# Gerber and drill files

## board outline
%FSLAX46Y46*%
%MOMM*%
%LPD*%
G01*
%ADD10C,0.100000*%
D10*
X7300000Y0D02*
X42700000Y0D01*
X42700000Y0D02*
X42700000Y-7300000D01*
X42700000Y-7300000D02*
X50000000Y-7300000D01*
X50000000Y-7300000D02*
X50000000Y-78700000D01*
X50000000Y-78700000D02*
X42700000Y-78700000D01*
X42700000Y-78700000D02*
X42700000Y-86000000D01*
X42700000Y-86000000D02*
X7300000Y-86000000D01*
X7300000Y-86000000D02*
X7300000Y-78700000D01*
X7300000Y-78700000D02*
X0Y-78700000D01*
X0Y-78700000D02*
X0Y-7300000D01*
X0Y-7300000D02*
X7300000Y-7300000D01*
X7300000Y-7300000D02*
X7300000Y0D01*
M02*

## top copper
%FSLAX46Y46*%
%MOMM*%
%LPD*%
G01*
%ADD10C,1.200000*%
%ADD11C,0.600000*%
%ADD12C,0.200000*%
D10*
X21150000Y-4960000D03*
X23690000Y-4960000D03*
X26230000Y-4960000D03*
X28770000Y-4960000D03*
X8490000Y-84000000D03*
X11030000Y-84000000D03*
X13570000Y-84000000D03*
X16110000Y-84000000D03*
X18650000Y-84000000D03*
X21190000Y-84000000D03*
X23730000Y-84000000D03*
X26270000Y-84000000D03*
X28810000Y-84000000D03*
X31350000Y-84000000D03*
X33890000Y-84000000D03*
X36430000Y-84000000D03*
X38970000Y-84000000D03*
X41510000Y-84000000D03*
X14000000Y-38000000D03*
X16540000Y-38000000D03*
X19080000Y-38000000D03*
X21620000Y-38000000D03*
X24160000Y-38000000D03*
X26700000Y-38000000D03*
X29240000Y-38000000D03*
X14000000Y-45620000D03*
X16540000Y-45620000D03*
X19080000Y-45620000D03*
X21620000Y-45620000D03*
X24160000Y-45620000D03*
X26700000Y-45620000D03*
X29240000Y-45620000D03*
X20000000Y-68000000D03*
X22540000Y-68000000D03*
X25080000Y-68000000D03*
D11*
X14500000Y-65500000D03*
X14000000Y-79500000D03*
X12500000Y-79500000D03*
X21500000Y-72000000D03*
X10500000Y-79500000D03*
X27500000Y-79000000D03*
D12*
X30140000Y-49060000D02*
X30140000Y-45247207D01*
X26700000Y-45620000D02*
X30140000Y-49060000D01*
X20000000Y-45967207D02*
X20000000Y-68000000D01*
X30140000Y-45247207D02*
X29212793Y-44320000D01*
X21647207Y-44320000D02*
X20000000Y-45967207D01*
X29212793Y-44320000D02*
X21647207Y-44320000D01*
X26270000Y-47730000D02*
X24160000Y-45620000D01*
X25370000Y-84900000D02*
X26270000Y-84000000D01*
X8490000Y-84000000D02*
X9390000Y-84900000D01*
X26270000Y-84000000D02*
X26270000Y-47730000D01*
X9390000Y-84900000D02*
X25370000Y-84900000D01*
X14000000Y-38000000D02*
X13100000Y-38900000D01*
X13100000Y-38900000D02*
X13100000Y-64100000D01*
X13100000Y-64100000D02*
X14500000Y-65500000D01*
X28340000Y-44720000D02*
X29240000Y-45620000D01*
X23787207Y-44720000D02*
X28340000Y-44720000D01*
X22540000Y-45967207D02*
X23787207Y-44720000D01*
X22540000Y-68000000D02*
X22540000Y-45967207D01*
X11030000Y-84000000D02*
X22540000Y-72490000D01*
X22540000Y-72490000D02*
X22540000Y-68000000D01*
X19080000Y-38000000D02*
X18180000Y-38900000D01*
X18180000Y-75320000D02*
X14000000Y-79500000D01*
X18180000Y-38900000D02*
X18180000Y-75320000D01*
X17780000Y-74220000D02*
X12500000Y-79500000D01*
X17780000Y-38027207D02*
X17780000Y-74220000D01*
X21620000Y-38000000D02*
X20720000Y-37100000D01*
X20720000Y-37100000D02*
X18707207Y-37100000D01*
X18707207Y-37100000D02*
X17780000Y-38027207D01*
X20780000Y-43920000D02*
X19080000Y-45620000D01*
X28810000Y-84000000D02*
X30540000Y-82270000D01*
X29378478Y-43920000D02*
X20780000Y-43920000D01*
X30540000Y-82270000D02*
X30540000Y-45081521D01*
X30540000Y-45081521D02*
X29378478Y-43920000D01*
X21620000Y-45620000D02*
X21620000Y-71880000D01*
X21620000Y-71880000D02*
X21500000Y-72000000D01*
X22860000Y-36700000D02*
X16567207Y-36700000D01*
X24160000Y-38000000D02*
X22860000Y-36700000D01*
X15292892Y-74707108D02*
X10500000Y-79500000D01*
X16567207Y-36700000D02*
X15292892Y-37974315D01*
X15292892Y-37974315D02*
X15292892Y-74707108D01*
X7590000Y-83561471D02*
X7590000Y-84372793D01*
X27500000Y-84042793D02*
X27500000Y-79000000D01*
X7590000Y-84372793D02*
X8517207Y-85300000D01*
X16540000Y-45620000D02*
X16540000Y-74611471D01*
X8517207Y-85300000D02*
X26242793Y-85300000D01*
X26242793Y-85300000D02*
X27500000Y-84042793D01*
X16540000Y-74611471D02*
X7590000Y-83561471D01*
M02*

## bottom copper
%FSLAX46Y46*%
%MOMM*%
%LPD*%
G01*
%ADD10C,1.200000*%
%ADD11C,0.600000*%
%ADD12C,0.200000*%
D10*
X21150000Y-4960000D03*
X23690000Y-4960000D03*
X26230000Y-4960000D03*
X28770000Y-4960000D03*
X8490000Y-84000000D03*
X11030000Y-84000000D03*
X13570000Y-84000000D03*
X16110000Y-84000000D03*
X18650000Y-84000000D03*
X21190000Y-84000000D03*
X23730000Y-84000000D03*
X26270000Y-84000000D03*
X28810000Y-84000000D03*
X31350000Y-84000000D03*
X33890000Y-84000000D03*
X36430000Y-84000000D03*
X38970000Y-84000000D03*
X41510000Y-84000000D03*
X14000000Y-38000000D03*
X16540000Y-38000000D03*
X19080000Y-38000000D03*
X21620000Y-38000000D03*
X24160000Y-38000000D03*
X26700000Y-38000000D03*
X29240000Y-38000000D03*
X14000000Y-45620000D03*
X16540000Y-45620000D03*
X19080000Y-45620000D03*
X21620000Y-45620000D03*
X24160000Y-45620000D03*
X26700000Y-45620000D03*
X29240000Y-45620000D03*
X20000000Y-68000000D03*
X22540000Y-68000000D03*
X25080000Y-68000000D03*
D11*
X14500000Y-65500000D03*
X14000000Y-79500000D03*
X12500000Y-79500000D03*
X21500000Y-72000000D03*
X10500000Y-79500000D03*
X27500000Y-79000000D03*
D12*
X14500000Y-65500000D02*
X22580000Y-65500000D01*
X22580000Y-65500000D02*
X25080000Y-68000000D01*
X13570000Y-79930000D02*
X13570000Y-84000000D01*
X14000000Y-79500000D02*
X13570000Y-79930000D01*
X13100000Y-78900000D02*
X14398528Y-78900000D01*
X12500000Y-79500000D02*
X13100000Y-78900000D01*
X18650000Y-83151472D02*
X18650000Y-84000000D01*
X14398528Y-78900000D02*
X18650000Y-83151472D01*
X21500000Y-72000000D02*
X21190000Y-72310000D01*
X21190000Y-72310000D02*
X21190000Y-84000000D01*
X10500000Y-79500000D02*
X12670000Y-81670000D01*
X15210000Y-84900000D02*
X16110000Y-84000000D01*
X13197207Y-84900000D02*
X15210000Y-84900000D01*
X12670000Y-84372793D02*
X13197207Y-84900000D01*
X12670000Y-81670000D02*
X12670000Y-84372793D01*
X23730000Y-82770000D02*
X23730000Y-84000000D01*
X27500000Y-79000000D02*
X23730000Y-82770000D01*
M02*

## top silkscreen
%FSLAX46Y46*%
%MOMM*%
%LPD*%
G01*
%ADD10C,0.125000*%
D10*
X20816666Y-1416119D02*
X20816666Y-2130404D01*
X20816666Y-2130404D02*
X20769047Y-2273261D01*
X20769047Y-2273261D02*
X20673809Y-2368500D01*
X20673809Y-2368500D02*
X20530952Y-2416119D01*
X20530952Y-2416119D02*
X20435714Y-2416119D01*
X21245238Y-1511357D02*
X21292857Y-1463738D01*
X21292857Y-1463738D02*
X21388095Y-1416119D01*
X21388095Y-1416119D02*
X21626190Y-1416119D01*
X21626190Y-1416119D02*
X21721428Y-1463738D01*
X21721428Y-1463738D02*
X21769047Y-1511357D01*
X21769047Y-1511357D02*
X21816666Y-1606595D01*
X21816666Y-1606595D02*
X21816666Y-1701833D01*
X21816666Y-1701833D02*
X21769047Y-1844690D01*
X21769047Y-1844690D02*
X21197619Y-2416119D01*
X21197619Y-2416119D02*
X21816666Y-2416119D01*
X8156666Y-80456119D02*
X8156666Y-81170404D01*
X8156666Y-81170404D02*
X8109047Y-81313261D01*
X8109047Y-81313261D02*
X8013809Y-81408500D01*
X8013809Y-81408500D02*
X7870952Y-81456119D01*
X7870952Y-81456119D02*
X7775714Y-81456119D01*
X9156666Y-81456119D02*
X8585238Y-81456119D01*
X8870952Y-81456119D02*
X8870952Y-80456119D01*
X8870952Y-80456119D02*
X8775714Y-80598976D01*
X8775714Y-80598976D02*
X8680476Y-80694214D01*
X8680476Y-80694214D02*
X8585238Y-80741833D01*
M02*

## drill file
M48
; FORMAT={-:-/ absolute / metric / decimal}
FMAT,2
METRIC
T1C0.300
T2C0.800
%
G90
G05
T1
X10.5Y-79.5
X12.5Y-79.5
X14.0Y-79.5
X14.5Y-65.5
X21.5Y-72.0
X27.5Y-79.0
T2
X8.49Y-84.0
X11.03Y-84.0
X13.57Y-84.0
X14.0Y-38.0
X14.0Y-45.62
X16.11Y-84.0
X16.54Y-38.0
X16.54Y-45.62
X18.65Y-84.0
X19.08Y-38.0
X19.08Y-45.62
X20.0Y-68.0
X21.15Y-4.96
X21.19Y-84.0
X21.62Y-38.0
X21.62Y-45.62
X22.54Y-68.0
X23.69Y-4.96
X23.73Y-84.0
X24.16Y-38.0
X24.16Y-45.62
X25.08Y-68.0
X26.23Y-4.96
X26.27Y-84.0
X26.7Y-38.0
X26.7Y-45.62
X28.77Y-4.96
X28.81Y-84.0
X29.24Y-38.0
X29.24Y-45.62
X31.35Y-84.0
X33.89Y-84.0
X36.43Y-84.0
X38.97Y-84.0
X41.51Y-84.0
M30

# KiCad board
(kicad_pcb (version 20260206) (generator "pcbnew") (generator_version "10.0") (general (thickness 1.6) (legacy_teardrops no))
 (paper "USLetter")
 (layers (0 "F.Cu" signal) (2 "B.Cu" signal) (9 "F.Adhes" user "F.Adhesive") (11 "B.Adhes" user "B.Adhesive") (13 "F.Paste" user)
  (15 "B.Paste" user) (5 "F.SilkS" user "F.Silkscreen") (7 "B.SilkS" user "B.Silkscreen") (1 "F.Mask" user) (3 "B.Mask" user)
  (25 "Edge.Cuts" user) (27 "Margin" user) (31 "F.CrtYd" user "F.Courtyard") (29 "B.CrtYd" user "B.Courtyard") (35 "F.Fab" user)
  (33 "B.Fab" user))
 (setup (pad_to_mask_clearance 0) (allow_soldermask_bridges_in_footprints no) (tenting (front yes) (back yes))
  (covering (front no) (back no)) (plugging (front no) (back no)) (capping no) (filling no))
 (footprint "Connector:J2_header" (layer "F.Cu") (at 21.15 4.96)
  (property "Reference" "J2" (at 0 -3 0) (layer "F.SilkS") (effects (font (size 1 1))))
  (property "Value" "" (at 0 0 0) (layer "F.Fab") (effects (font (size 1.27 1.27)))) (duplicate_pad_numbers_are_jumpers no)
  (pad "1" thru_hole circle (at 0 0) (size 1.2 1.2) (drill 0.8) (layers "*.Cu" "*.Mask") (remove_unused_layers no))
  (pad "2" thru_hole circle (at 2.54 0) (size 1.2 1.2) (drill 0.8) (layers "*.Cu" "*.Mask") (remove_unused_layers no))
  (pad "3" thru_hole circle (at 5.08 0) (size 1.2 1.2) (drill 0.8) (layers "*.Cu" "*.Mask") (remove_unused_layers no))
  (pad "4" thru_hole circle (at 7.62 0) (size 1.2 1.2) (drill 0.8) (layers "*.Cu" "*.Mask") (remove_unused_layers no)))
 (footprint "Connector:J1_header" (layer "F.Cu") (at 8.49 84)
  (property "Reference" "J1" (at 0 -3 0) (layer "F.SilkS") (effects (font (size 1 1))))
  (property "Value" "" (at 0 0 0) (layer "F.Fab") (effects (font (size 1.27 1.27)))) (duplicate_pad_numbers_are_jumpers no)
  (pad "1" thru_hole circle (at 0 0) (size 1.2 1.2) (drill 0.8) (layers "*.Cu" "*.Mask") (remove_unused_layers no) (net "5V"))
  (pad "2" thru_hole circle (at 2.54 0) (size 1.2 1.2) (drill 0.8) (layers "*.Cu" "*.Mask") (remove_unused_layers no) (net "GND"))
  (pad "3" thru_hole circle (at 5.08 0) (size 1.2 1.2) (drill 0.8) (layers "*.Cu" "*.Mask") (remove_unused_layers no) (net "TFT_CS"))
  (pad "4" thru_hole circle (at 7.62 0) (size 1.2 1.2) (drill 0.8) (layers "*.Cu" "*.Mask") (remove_unused_layers no) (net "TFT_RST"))
  (pad "5" thru_hole circle (at 10.16 0) (size 1.2 1.2) (drill 0.8) (layers "*.Cu" "*.Mask") (remove_unused_layers no) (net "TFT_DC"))
  (pad "6" thru_hole circle (at 12.7 0) (size 1.2 1.2) (drill 0.8) (layers "*.Cu" "*.Mask") (remove_unused_layers no) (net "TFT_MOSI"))
  (pad "7" thru_hole circle (at 15.24 0) (size 1.2 1.2) (drill 0.8) (layers "*.Cu" "*.Mask") (remove_unused_layers no) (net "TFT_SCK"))
  (pad "8" thru_hole circle (at 17.78 0) (size 1.2 1.2) (drill 0.8) (layers "*.Cu" "*.Mask") (remove_unused_layers no) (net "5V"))
  (pad "9" thru_hole circle (at 20.32 0) (size 1.2 1.2) (drill 0.8) (layers "*.Cu" "*.Mask") (remove_unused_layers no) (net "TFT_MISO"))
  (pad "10" thru_hole circle (at 22.86 0) (size 1.2 1.2) (drill 0.8) (layers "*.Cu" "*.Mask") (remove_unused_layers no))
  (pad "11" thru_hole circle (at 25.4 0) (size 1.2 1.2) (drill 0.8) (layers "*.Cu" "*.Mask") (remove_unused_layers no))
  (pad "12" thru_hole circle (at 27.94 0) (size 1.2 1.2) (drill 0.8) (layers "*.Cu" "*.Mask") (remove_unused_layers no))
  (pad "13" thru_hole circle (at 30.48 0) (size 1.2 1.2) (drill 0.8) (layers "*.Cu" "*.Mask") (remove_unused_layers no))
  (pad "14" thru_hole circle (at 33.02 0) (size 1.2 1.2) (drill 0.8) (layers "*.Cu" "*.Mask") (remove_unused_layers no)))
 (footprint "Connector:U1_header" (layer "B.Cu") (at 14 38)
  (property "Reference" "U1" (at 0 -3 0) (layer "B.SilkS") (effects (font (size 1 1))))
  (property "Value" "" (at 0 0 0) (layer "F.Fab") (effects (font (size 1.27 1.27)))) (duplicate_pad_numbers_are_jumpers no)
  (pad "1" thru_hole circle (at 0 0) (size 1.2 1.2) (drill 0.8) (layers "*.Cu" "*.Mask") (remove_unused_layers no) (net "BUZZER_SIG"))
  (pad "2" thru_hole circle (at 2.54 0) (size 1.2 1.2) (drill 0.8) (layers "*.Cu" "*.Mask") (remove_unused_layers no))
  (pad "3" thru_hole circle (at 5.08 0) (size 1.2 1.2) (drill 0.8) (layers "*.Cu" "*.Mask") (remove_unused_layers no) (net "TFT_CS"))
  (pad "4" thru_hole circle (at 7.62 0) (size 1.2 1.2) (drill 0.8) (layers "*.Cu" "*.Mask") (remove_unused_layers no) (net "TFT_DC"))
  (pad "5" thru_hole circle (at 10.16 0) (size 1.2 1.2) (drill 0.8) (layers "*.Cu" "*.Mask") (remove_unused_layers no) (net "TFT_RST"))
  (pad "6" thru_hole circle (at 12.7 0) (size 1.2 1.2) (drill 0.8) (layers "*.Cu" "*.Mask") (remove_unused_layers no))
  (pad "7" thru_hole circle (at 15.24 0) (size 1.2 1.2) (drill 0.8) (layers "*.Cu" "*.Mask") (remove_unused_layers no))
  (pad "8" thru_hole circle (at 0 7.62) (size 1.2 1.2) (drill 0.8) (layers "*.Cu" "*.Mask") (remove_unused_layers no))
  (pad "9" thru_hole circle (at 2.54 7.62) (size 1.2 1.2) (drill 0.8) (layers "*.Cu" "*.Mask") (remove_unused_layers no) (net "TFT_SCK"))
  (pad "10" thru_hole circle (at 5.08 7.62) (size 1.2 1.2) (drill 0.8) (layers "*.Cu" "*.Mask") (remove_unused_layers no) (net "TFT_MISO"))
  (pad "11" thru_hole circle (at 7.62 7.62) (size 1.2 1.2) (drill 0.8) (layers "*.Cu" "*.Mask") (remove_unused_layers no) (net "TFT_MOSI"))
  (pad "12" thru_hole circle (at 10.16 7.62) (size 1.2 1.2) (drill 0.8) (layers "*.Cu" "*.Mask") (remove_unused_layers no) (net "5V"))
  (pad "13" thru_hole circle (at 12.7 7.62) (size 1.2 1.2) (drill 0.8) (layers "*.Cu" "*.Mask") (remove_unused_layers no) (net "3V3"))
  (pad "14" thru_hole circle (at 15.24 7.62) (size 1.2 1.2) (drill 0.8) (layers "*.Cu" "*.Mask") (remove_unused_layers no) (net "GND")))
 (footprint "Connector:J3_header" (layer "B.Cu") (at 20 68)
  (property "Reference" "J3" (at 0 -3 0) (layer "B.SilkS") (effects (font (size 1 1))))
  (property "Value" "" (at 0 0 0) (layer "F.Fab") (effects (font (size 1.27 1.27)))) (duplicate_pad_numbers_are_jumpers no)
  (pad "1" thru_hole circle (at 0 0) (size 1.2 1.2) (drill 0.8) (layers "*.Cu" "*.Mask") (remove_unused_layers no) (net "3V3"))
  (pad "2" thru_hole circle (at 2.54 0) (size 1.2 1.2) (drill 0.8) (layers "*.Cu" "*.Mask") (remove_unused_layers no) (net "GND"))
  (pad "3" thru_hole circle (at 5.08 0) (size 1.2 1.2) (drill 0.8) (layers "*.Cu" "*.Mask") (remove_unused_layers no) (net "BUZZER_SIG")))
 (gr_line (start 7.3 0) (end 42.7 0) (stroke (width 0.1) (type default)) (layer "Edge.Cuts"))
 (gr_line (start 42.7 0) (end 42.7 7.3) (stroke (width 0.1) (type default)) (layer "Edge.Cuts"))
 (gr_line (start 42.7 7.3) (end 50 7.3) (stroke (width 0.1) (type default)) (layer "Edge.Cuts"))
 (gr_line (start 50 7.3) (end 50 78.7) (stroke (width 0.1) (type default)) (layer "Edge.Cuts"))
 (gr_line (start 50 78.7) (end 42.7 78.7) (stroke (width 0.1) (type default)) (layer "Edge.Cuts"))
 (gr_line (start 42.7 78.7) (end 42.7 86) (stroke (width 0.1) (type default)) (layer "Edge.Cuts"))
 (gr_line (start 42.7 86) (end 7.3 86) (stroke (width 0.1) (type default)) (layer "Edge.Cuts"))
 (gr_line (start 7.3 86) (end 7.3 78.7) (stroke (width 0.1) (type default)) (layer "Edge.Cuts"))
 (gr_line (start 7.3 78.7) (end 0 78.7) (stroke (width 0.1) (type default)) (layer "Edge.Cuts"))
 (gr_line (start 0 78.7) (end 0 7.3) (stroke (width 0.1) (type default)) (layer "Edge.Cuts"))
 (gr_line (start 0 7.3) (end 7.3 7.3) (stroke (width 0.1) (type default)) (layer "Edge.Cuts"))
 (gr_line (start 7.3 7.3) (end 7.3 0) (stroke (width 0.1) (type default)) (layer "Edge.Cuts"))
 (segment (start 30.14 49.06) (end 30.14 45.247207) (width 0.2) (layer "F.Cu") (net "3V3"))
 (segment (start 26.7 45.62) (end 30.14 49.06) (width 0.2) (layer "F.Cu") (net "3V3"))
 (segment (start 20 45.967207) (end 20 68) (width 0.2) (layer "F.Cu") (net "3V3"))
 (segment (start 30.14 45.247207) (end 29.212793 44.32) (width 0.2) (layer "F.Cu") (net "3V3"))
 (segment (start 21.647207 44.32) (end 20 45.967207) (width 0.2) (layer "F.Cu") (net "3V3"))
 (segment (start 29.212793 44.32) (end 21.647207 44.32) (width 0.2) (layer "F.Cu") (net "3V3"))
 (segment (start 26.27 47.73) (end 24.16 45.62) (width 0.2) (layer "F.Cu") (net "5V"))
 (segment (start 25.37 84.9) (end 26.27 84) (width 0.2) (layer "F.Cu") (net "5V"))
 (segment (start 8.49 84) (end 9.39 84.9) (width 0.2) (layer "F.Cu") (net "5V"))
 (segment (start 26.27 84) (end 26.27 47.73) (width 0.2) (layer "F.Cu") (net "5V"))
 (segment (start 9.39 84.9) (end 25.37 84.9) (width 0.2) (layer "F.Cu") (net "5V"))
 (segment (start 14 38) (end 13.1 38.9) (width 0.2) (layer "F.Cu") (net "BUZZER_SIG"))
 (segment (start 13.1 38.9) (end 13.1 64.1) (width 0.2) (layer "F.Cu") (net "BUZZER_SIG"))
 (segment (start 13.1 64.1) (end 14.5 65.5) (width 0.2) (layer "F.Cu") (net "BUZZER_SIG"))
 (via (at 14.5 65.5) (size 0.6) (drill 0.3) (layers "F.Cu" "B.Cu") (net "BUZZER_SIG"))
 (segment (start 14.5 65.5) (end 22.58 65.5) (width 0.2) (layer "B.Cu") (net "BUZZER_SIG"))
 (segment (start 22.58 65.5) (end 25.08 68) (width 0.2) (layer "B.Cu") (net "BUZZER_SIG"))
 (segment (start 28.34 44.72) (end 29.24 45.62) (width 0.2) (layer "F.Cu") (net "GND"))
 (segment (start 23.787207 44.72) (end 28.34 44.72) (width 0.2) (layer "F.Cu") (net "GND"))
 (segment (start 22.54 45.967207) (end 23.787207 44.72) (width 0.2) (layer "F.Cu") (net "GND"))
 (segment (start 22.54 68) (end 22.54 45.967207) (width 0.2) (layer "F.Cu") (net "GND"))
 (segment (start 11.03 84) (end 22.54 72.49) (width 0.2) (layer "F.Cu") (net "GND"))
 (segment (start 22.54 72.49) (end 22.54 68) (width 0.2) (layer "F.Cu") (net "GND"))
 (segment (start 19.08 38) (end 18.18 38.9) (width 0.2) (layer "F.Cu") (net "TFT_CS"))
 (segment (start 18.18 75.32) (end 14 79.5) (width 0.2) (layer "F.Cu") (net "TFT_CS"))
 (segment (start 18.18 38.9) (end 18.18 75.32) (width 0.2) (layer "F.Cu") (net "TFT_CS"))
 (via (at 14 79.5) (size 0.6) (drill 0.3) (layers "F.Cu" "B.Cu") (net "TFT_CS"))
 (segment (start 13.57 79.93) (end 13.57 84) (width 0.2) (layer "B.Cu") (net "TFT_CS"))
 (segment (start 14 79.5) (end 13.57 79.93) (width 0.2) (layer "B.Cu") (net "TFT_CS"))
 (segment (start 17.78 74.22) (end 12.5 79.5) (width 0.2) (layer "F.Cu") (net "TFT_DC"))
 (segment (start 17.78 38.027207) (end 17.78 74.22) (width 0.2) (layer "F.Cu") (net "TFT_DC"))
 (segment (start 21.62 38) (end 20.72 37.1) (width 0.2) (layer "F.Cu") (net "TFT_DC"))
 (segment (start 20.72 37.1) (end 18.707207 37.1) (width 0.2) (layer "F.Cu") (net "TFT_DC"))
 (segment (start 18.707207 37.1) (end 17.78 38.027207) (width 0.2) (layer "F.Cu") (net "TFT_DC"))
 (via (at 12.5 79.5) (size 0.6) (drill 0.3) (layers "F.Cu" "B.Cu") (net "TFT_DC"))
 (segment (start 13.1 78.9) (end 14.398528 78.9) (width 0.2) (layer "B.Cu") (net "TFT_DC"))
 (segment (start 12.5 79.5) (end 13.1 78.9) (width 0.2) (layer "B.Cu") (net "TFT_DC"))
 (segment (start 18.65 83.151472) (end 18.65 84) (width 0.2) (layer "B.Cu") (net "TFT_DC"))
 (segment (start 14.398528 78.9) (end 18.65 83.151472) (width 0.2) (layer "B.Cu") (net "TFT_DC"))
 (segment (start 20.78 43.92) (end 19.08 45.62) (width 0.2) (layer "F.Cu") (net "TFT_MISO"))
 (segment (start 28.81 84) (end 30.54 82.27) (width 0.2) (layer "F.Cu") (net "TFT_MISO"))
 (segment (start 29.378478 43.92) (end 20.78 43.92) (width 0.2) (layer "F.Cu") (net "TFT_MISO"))
 (segment (start 30.54 82.27) (end 30.54 45.081521) (width 0.2) (layer "F.Cu") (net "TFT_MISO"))
 (segment (start 30.54 45.081521) (end 29.378478 43.92) (width 0.2) (layer "F.Cu") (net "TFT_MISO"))
 (segment (start 21.62 45.62) (end 21.62 71.88) (width 0.2) (layer "F.Cu") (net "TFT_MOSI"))
 (segment (start 21.62 71.88) (end 21.5 72) (width 0.2) (layer "F.Cu") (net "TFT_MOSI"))
 (via (at 21.5 72) (size 0.6) (drill 0.3) (layers "F.Cu" "B.Cu") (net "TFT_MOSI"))
 (segment (start 21.5 72) (end 21.19 72.31) (width 0.2) (layer "B.Cu") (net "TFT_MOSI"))
 (segment (start 21.19 72.31) (end 21.19 84) (width 0.2) (layer "B.Cu") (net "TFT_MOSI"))
 (segment (start 22.86 36.7) (end 16.567207 36.7) (width 0.2) (layer "F.Cu") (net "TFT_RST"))
 (segment (start 24.16 38) (end 22.86 36.7) (width 0.2) (layer "F.Cu") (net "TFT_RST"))
 (segment (start 15.292892 74.707108) (end 10.5 79.5) (width 0.2) (layer "F.Cu") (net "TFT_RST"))
 (segment (start 16.567207 36.7) (end 15.292892 37.974315) (width 0.2) (layer "F.Cu") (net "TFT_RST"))
 (segment (start 15.292892 37.974315) (end 15.292892 74.707108) (width 0.2) (layer "F.Cu") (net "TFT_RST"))
 (via (at 10.5 79.5) (size 0.6) (drill 0.3) (layers "F.Cu" "B.Cu") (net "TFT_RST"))
 (segment (start 10.5 79.5) (end 12.67 81.67) (width 0.2) (layer "B.Cu") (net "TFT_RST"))
 (segment (start 15.21 84.9) (end 16.11 84) (width 0.2) (layer "B.Cu") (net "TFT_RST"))
 (segment (start 13.197207 84.9) (end 15.21 84.9) (width 0.2) (layer "B.Cu") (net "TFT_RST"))
 (segment (start 12.67 84.372793) (end 13.197207 84.9) (width 0.2) (layer "B.Cu") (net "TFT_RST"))
 (segment (start 12.67 81.67) (end 12.67 84.372793) (width 0.2) (layer "B.Cu") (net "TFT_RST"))
 (segment (start 7.59 83.561471) (end 7.59 84.372793) (width 0.2) (layer "F.Cu") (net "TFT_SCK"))
 (segment (start 27.5 84.042793) (end 27.5 79) (width 0.2) (layer "F.Cu") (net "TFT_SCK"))
 (segment (start 7.59 84.372793) (end 8.517207 85.3) (width 0.2) (layer "F.Cu") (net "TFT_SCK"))
 (segment (start 16.54 45.62) (end 16.54 74.611471) (width 0.2) (layer "F.Cu") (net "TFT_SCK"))
 (segment (start 8.517207 85.3) (end 26.242793 85.3) (width 0.2) (layer "F.Cu") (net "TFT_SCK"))
 (segment (start 26.242793 85.3) (end 27.5 84.042793) (width 0.2) (layer "F.Cu") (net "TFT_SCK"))
 (segment (start 16.54 74.611471) (end 7.59 83.561471) (width 0.2) (layer "F.Cu") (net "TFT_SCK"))
 (via (at 27.5 79) (size 0.6) (drill 0.3) (layers "F.Cu" "B.Cu") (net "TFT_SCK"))
 (segment (start 23.73 82.77) (end 23.73 84) (width 0.2) (layer "B.Cu") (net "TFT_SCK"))
 (segment (start 27.5 79) (end 23.73 82.77) (width 0.2) (layer "B.Cu") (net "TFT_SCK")))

